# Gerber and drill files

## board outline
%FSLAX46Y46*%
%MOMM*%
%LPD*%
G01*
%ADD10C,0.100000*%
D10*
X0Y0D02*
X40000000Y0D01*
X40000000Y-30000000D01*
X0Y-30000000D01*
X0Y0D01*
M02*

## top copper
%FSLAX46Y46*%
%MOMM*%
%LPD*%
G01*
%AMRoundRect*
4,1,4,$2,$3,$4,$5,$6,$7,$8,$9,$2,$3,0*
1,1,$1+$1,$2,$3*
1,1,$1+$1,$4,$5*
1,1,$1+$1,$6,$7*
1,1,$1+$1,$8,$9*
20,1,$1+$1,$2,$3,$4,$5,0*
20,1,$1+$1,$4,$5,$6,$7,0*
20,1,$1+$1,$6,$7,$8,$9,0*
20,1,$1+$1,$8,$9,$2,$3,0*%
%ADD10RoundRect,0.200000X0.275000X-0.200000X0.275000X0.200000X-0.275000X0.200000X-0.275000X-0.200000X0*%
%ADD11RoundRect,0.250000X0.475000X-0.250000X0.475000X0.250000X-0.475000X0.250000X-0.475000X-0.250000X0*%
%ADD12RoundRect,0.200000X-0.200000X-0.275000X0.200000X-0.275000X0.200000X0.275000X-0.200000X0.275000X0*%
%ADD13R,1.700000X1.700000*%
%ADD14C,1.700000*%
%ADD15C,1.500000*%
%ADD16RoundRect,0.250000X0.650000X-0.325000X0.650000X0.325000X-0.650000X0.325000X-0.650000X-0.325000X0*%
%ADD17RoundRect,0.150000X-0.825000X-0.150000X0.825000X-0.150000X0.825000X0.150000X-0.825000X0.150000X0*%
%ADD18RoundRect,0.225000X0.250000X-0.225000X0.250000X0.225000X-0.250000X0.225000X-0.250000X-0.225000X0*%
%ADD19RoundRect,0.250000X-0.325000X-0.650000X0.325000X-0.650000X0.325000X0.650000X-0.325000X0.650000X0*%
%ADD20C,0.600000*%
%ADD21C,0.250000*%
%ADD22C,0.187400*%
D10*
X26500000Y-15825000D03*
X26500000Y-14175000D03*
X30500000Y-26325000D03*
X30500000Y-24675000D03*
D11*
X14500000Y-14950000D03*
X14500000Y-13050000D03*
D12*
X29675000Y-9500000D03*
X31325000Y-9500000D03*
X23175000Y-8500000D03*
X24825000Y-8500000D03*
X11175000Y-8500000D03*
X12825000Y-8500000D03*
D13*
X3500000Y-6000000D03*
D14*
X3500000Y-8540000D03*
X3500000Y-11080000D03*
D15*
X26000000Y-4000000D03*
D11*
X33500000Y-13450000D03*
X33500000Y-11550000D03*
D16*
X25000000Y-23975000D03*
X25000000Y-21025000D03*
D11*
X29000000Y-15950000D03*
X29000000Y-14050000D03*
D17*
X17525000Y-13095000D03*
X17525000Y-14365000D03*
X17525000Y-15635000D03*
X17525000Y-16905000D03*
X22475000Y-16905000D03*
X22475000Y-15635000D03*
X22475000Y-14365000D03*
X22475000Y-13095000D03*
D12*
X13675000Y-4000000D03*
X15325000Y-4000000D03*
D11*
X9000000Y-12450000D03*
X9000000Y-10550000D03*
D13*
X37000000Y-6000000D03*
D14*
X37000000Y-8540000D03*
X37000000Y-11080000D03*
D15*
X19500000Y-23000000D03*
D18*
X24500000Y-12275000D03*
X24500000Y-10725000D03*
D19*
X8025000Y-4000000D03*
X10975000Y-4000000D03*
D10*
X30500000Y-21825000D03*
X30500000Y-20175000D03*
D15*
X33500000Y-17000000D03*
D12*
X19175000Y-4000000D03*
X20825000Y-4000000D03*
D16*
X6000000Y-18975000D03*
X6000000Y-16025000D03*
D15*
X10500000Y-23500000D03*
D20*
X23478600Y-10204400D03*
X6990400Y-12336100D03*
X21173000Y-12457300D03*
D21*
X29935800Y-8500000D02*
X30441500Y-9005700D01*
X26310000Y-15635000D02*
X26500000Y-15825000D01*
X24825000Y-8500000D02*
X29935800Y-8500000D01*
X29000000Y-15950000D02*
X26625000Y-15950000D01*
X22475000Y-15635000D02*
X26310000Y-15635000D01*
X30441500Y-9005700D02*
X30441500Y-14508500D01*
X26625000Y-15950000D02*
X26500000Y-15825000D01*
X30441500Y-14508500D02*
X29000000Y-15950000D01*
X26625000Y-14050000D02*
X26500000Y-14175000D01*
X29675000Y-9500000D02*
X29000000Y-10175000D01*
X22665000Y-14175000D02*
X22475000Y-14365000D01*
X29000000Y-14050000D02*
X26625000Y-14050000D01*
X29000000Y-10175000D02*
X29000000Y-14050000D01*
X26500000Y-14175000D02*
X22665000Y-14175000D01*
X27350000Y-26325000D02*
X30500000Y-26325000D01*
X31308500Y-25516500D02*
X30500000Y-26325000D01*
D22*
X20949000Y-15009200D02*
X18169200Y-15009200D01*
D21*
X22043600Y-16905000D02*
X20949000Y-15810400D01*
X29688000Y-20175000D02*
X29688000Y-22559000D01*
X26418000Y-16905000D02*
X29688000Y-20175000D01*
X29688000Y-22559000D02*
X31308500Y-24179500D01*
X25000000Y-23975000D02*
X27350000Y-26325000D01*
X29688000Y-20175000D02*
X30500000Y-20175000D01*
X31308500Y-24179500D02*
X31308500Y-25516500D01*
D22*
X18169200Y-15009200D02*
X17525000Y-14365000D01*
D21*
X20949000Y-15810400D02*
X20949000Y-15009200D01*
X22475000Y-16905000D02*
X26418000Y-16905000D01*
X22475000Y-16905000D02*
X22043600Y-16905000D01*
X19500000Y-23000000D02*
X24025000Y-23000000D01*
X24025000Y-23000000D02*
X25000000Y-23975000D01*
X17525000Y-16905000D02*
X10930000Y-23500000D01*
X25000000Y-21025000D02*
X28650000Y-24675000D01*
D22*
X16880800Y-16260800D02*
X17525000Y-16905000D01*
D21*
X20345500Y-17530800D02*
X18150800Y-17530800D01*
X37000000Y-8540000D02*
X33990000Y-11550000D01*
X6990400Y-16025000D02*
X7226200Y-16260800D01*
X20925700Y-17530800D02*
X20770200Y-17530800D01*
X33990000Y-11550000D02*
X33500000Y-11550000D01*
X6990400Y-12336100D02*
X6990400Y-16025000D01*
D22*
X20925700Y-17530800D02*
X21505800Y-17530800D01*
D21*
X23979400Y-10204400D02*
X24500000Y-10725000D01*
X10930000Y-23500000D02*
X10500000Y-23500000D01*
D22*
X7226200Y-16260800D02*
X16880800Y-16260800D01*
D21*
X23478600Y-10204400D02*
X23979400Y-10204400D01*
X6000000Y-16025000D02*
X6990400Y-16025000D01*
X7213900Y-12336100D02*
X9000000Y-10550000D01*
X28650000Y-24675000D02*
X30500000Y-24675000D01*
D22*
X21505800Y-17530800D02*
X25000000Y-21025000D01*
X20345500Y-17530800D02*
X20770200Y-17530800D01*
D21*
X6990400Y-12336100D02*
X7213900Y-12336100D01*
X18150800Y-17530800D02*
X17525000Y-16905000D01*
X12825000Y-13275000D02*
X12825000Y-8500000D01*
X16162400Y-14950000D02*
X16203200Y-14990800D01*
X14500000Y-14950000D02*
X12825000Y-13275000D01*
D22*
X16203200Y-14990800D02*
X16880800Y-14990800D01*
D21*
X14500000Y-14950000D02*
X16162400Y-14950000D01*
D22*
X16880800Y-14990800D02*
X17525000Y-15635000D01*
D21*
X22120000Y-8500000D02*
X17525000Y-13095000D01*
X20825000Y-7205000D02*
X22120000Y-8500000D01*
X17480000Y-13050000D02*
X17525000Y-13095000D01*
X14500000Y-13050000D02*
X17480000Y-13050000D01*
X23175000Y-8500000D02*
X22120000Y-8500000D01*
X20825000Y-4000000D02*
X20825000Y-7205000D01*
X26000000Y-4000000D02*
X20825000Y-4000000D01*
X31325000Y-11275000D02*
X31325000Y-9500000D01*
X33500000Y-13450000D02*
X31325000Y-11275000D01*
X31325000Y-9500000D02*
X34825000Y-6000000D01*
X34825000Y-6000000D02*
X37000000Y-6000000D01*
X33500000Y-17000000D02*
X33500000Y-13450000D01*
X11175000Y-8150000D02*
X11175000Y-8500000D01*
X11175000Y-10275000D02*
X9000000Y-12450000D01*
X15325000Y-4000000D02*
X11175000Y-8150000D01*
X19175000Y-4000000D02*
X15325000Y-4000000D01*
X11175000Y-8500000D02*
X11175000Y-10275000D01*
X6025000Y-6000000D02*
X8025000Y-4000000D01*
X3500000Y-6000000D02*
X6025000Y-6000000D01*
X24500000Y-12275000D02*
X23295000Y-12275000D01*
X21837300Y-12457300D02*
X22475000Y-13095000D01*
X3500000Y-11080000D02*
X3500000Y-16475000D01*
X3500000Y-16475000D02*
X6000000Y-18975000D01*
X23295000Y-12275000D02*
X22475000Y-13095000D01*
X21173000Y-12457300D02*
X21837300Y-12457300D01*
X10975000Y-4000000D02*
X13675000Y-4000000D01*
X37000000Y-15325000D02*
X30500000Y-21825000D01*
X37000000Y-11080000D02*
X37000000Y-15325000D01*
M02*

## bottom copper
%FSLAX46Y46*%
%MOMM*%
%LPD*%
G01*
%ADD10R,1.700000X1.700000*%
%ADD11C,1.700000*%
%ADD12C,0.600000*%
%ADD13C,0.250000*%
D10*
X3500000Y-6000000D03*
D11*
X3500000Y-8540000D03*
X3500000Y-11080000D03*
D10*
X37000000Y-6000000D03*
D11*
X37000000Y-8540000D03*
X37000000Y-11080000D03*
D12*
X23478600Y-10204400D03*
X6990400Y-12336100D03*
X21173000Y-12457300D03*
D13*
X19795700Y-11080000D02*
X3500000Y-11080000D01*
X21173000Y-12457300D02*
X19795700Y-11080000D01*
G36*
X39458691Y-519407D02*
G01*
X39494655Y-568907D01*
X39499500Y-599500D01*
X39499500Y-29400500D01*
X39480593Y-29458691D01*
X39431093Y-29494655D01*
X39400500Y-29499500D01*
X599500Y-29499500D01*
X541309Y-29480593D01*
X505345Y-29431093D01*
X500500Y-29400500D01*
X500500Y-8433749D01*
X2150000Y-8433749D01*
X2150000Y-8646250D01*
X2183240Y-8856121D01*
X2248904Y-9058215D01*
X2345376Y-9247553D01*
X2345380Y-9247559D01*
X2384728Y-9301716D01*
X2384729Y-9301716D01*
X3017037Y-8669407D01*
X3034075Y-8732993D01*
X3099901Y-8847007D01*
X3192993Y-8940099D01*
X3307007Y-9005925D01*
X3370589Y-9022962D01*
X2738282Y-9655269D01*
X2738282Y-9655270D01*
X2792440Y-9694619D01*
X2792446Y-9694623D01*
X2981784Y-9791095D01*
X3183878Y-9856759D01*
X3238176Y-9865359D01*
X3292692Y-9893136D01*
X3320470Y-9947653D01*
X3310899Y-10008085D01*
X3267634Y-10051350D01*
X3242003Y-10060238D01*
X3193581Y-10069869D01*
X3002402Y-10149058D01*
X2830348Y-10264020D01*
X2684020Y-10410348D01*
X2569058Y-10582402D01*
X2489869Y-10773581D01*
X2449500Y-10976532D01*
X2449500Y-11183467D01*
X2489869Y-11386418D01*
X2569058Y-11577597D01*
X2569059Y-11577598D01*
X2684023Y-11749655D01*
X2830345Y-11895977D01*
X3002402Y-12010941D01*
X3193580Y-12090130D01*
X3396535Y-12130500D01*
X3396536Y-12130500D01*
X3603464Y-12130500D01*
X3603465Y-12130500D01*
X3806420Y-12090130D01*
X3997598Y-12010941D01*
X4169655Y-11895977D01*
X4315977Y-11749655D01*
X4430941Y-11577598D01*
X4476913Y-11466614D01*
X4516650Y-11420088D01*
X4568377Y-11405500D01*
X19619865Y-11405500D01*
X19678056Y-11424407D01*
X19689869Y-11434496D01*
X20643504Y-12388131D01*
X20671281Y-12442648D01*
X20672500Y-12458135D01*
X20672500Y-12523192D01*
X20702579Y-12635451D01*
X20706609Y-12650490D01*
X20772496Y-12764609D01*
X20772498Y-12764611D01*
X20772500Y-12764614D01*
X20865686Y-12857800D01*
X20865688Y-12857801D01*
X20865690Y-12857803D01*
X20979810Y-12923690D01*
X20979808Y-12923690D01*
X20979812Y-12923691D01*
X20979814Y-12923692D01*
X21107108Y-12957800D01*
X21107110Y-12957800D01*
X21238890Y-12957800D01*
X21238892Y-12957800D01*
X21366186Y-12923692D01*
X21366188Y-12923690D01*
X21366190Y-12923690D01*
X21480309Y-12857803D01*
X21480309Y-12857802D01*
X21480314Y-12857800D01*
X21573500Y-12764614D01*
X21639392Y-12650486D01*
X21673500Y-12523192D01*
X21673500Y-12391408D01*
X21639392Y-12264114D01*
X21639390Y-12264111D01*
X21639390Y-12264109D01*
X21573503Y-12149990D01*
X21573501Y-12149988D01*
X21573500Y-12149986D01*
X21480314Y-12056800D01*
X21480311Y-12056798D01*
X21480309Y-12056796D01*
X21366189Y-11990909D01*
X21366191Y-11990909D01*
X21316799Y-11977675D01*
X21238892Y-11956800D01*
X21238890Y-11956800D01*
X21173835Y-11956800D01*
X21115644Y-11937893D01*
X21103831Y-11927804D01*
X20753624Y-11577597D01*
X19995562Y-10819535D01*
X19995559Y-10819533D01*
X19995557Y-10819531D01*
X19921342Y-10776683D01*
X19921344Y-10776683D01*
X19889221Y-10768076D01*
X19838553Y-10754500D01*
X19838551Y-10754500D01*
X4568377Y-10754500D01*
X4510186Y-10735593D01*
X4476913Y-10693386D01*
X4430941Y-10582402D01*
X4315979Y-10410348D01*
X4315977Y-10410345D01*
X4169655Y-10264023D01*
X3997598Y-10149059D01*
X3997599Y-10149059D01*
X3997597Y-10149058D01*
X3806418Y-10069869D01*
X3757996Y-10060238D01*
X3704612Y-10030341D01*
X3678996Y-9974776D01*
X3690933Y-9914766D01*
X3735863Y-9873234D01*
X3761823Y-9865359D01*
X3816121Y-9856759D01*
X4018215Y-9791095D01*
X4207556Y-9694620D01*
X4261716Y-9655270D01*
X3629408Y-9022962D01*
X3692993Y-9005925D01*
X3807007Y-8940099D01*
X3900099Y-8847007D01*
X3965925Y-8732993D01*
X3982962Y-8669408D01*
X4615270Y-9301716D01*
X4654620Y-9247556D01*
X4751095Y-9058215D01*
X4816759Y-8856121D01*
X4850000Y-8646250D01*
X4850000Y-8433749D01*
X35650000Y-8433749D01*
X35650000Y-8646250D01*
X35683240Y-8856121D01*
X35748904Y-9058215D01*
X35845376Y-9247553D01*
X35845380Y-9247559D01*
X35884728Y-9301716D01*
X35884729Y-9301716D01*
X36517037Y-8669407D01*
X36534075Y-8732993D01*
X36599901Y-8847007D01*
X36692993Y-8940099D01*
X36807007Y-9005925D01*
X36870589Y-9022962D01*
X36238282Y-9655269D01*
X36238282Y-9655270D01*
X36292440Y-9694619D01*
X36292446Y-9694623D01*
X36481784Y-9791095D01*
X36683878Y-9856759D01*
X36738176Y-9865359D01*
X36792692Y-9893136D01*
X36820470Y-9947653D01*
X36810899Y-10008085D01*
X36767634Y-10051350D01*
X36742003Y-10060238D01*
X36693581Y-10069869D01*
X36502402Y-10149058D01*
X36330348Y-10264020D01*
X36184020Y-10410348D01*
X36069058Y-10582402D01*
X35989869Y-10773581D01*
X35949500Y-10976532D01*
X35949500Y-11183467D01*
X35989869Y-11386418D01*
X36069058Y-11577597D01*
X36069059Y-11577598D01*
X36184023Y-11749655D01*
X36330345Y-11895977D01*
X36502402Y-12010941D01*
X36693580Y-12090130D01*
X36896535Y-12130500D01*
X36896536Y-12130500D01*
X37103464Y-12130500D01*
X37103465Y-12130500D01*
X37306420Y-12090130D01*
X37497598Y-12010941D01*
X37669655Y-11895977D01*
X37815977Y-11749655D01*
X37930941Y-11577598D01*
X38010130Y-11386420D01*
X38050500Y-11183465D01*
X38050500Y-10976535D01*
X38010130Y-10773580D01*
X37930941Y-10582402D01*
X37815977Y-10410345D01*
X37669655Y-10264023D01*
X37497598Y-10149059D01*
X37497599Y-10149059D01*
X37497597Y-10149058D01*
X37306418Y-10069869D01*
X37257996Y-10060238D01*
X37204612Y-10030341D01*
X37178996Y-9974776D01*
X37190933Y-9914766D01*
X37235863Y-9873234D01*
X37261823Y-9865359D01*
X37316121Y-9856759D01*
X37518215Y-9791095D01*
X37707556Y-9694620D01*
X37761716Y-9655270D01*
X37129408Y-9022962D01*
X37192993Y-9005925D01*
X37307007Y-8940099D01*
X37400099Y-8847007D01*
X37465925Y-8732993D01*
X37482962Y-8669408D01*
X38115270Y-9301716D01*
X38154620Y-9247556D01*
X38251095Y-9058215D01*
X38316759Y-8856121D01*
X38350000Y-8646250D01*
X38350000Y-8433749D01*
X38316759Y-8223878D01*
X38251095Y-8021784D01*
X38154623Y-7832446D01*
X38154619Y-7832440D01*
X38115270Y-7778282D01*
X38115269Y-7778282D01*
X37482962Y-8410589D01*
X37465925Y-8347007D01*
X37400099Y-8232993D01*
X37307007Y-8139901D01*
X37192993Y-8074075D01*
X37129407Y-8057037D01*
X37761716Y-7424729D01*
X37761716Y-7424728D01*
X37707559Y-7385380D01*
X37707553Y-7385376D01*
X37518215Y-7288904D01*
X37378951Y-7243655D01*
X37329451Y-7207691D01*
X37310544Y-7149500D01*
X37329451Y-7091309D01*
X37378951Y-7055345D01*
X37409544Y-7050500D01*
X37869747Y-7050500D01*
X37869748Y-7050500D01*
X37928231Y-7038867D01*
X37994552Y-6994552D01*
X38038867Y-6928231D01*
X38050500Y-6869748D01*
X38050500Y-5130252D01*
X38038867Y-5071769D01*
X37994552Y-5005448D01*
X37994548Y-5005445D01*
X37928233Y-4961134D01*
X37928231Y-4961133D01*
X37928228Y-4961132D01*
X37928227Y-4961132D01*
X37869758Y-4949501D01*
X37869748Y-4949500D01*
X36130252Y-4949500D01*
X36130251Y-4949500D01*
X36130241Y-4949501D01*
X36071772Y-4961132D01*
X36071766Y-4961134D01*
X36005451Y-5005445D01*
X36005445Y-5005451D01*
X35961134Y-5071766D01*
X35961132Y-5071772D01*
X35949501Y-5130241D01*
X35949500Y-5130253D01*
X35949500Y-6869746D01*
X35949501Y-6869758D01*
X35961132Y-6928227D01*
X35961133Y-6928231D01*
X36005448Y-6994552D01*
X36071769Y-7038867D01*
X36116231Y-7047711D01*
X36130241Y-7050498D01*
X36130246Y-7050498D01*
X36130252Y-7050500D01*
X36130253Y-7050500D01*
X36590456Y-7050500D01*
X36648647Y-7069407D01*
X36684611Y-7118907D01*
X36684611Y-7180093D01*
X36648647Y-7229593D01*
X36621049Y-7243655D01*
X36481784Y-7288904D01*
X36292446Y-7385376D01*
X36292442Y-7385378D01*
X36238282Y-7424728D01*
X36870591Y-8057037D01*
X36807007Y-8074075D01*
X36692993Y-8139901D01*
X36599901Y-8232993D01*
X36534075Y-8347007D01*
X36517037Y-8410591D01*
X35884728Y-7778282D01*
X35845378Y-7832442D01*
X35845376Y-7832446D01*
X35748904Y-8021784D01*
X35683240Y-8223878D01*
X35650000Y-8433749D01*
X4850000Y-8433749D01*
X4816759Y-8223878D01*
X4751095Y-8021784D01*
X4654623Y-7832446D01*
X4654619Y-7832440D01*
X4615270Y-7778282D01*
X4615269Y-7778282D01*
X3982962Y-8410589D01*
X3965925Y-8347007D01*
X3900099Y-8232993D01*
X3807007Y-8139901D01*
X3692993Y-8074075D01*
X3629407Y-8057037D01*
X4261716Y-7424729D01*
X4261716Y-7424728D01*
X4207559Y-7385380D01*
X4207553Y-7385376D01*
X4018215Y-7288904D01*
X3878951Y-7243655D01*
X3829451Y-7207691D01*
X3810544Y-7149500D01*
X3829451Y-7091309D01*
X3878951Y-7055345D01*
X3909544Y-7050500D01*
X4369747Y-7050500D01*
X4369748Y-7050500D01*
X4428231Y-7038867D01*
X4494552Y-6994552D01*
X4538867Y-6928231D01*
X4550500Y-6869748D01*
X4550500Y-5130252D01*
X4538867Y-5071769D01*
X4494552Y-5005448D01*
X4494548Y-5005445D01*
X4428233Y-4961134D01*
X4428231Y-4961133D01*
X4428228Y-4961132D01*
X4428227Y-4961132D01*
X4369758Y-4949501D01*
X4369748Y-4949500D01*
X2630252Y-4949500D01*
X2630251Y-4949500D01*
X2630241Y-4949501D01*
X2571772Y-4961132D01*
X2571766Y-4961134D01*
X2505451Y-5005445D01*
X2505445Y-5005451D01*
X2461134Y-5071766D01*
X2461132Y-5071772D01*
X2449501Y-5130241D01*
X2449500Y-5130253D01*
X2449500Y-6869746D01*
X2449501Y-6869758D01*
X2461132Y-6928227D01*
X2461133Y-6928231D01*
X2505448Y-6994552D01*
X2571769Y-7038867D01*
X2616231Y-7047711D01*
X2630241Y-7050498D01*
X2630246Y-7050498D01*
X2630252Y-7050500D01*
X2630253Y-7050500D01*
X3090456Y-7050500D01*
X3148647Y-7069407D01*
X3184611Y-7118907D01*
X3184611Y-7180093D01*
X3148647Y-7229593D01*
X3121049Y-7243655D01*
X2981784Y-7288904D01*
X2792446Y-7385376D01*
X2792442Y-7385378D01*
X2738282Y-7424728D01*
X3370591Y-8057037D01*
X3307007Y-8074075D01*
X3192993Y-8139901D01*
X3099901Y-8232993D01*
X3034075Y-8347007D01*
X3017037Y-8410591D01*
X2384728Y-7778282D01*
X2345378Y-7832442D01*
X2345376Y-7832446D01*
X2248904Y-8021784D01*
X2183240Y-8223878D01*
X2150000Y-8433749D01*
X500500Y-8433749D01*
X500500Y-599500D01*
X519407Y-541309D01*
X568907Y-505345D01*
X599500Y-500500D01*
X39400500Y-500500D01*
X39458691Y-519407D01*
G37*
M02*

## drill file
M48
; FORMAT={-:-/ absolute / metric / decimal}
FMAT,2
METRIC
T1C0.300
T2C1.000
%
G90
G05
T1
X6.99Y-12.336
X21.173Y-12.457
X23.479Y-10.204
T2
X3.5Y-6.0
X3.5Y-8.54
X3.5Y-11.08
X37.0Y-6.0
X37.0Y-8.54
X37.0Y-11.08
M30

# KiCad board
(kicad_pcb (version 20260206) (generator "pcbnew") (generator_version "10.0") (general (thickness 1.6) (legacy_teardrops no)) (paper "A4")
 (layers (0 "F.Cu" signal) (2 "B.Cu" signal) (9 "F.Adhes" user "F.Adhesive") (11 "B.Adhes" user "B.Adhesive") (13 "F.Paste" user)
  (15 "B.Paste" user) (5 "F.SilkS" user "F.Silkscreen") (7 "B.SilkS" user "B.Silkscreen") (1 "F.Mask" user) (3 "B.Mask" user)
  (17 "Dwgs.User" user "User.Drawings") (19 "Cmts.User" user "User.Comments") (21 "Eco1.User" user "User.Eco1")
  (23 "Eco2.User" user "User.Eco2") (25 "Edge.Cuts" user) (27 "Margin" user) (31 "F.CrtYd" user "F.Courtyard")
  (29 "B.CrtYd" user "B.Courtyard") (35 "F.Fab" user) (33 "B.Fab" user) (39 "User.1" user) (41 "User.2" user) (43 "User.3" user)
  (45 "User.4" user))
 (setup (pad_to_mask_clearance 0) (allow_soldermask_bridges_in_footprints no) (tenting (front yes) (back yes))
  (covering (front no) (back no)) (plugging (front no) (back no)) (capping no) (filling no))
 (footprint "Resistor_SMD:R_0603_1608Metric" (layer "F.Cu") (at 26.5 15 90)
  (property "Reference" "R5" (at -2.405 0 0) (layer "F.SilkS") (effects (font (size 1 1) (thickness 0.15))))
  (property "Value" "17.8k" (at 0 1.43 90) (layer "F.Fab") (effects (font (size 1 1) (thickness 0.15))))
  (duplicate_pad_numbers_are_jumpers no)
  (pad "1" smd roundrect (at -0.825 0 90) (size 0.8 0.95) (layers "F.Cu" "F.Mask" "F.Paste") (roundrect_rratio 0.25) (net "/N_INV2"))
  (pad "2" smd roundrect (at 0.825 0 90) (size 0.8 0.95) (layers "F.Cu" "F.Mask" "F.Paste") (roundrect_rratio 0.25) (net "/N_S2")))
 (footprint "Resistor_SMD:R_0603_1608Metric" (layer "F.Cu") (at 30.5 25.5 90)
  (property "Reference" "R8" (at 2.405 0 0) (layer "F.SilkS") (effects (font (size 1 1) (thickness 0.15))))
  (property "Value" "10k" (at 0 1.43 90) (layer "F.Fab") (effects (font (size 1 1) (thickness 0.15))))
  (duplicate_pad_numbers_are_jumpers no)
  (pad "1" smd roundrect (at -0.825 0 90) (size 0.8 0.95) (layers "F.Cu" "F.Mask" "F.Paste") (roundrect_rratio 0.25) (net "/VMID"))
  (pad "2" smd roundrect (at 0.825 0 90) (size 0.8 0.95) (layers "F.Cu" "F.Mask" "F.Paste") (roundrect_rratio 0.25) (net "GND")))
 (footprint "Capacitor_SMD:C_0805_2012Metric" (layer "F.Cu") (at 14.5 14 90)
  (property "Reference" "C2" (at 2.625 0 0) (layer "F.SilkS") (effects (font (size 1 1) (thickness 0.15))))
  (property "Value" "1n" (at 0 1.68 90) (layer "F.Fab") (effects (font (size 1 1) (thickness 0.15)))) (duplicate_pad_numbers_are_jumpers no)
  (pad "1" smd roundrect (at -0.95 0 90) (size 1 1.45) (layers "F.Cu" "F.Mask" "F.Paste") (roundrect_rratio 0.25) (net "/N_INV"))
  (pad "2" smd roundrect (at 0.95 0 90) (size 1 1.45) (layers "F.Cu" "F.Mask" "F.Paste") (roundrect_rratio 0.25) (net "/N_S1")))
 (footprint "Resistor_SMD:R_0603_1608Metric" (layer "F.Cu") (at 30.5 9.5)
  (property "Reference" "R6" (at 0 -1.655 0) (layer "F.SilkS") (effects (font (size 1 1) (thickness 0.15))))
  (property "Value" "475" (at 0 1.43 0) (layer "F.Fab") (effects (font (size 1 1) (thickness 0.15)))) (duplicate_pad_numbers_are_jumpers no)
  (pad "1" smd roundrect (at -0.825 0) (size 0.8 0.95) (layers "F.Cu" "F.Mask" "F.Paste") (roundrect_rratio 0.25) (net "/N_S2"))
  (pad "2" smd roundrect (at 0.825 0) (size 0.8 0.95) (layers "F.Cu" "F.Mask" "F.Paste") (roundrect_rratio 0.25) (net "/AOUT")))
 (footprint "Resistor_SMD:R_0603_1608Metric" (layer "F.Cu") (at 24 8.5)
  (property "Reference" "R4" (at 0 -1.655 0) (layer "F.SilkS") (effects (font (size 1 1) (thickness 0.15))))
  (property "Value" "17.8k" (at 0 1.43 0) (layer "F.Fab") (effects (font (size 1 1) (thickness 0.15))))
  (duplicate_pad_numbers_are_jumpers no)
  (pad "1" smd roundrect (at -0.825 0) (size 0.8 0.95) (layers "F.Cu" "F.Mask" "F.Paste") (roundrect_rratio 0.25) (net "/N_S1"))
  (pad "2" smd roundrect (at 0.825 0) (size 0.8 0.95) (layers "F.Cu" "F.Mask" "F.Paste") (roundrect_rratio 0.25) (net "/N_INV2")))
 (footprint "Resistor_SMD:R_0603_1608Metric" (layer "F.Cu") (at 12 8.5)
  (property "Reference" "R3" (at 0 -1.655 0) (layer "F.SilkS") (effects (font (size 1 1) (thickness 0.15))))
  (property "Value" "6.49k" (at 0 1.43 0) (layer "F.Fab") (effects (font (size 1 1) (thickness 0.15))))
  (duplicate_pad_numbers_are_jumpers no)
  (pad "1" smd roundrect (at -0.825 0) (size 0.8 0.95) (layers "F.Cu" "F.Mask" "F.Paste") (roundrect_rratio 0.25) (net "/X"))
  (pad "2" smd roundrect (at 0.825 0) (size 0.8 0.95) (layers "F.Cu" "F.Mask" "F.Paste") (roundrect_rratio 0.25) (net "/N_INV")))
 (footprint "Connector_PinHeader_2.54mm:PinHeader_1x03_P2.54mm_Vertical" (layer "F.Cu") (at 3.5 6)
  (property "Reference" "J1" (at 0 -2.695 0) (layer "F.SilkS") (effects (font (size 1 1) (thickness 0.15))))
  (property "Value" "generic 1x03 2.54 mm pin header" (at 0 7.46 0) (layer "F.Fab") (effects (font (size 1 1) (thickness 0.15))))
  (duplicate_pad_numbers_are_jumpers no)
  (pad "1" thru_hole rect (at 0 0) (size 1.7 1.7) (drill 1) (layers "*.Cu" "*.Mask") (remove_unused_layers no) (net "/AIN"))
  (pad "2" thru_hole circle (at 0 2.54) (size 1.7 1.7) (drill 1) (layers "*.Cu" "*.Mask") (remove_unused_layers no) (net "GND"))
  (pad "3" thru_hole circle (at 0 5.08) (size 1.7 1.7) (drill 1) (layers "*.Cu" "*.Mask") (remove_unused_layers no) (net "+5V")))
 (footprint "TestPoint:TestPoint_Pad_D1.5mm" (layer "F.Cu") (at 26 4)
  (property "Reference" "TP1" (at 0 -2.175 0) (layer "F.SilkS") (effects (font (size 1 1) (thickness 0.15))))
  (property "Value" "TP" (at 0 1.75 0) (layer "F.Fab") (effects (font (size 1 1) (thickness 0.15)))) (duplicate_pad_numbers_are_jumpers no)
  (pad "1" smd circle (at 0 0) (size 1.5 1.5) (layers "F.Cu" "F.Mask") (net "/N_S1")))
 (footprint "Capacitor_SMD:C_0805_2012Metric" (layer "F.Cu") (at 33.5 12.5 90)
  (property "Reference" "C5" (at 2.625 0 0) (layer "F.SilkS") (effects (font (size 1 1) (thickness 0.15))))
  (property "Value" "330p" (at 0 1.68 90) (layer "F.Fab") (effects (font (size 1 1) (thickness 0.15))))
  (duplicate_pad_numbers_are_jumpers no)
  (pad "1" smd roundrect (at -0.95 0 90) (size 1 1.45) (layers "F.Cu" "F.Mask" "F.Paste") (roundrect_rratio 0.25) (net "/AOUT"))
  (pad "2" smd roundrect (at 0.95 0 90) (size 1 1.45) (layers "F.Cu" "F.Mask" "F.Paste") (roundrect_rratio 0.25) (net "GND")))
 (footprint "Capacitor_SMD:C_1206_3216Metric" (layer "F.Cu") (at 25 22.5 90)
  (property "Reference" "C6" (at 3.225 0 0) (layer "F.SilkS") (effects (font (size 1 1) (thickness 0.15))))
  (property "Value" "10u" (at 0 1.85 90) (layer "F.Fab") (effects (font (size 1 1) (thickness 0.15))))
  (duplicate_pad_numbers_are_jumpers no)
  (pad "1" smd roundrect (at -1.475 0 90) (size 1.15 1.8) (layers "F.Cu" "F.Mask" "F.Paste") (roundrect_rratio 0.217391) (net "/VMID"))
  (pad "2" smd roundrect (at 1.475 0 90) (size 1.15 1.8) (layers "F.Cu" "F.Mask" "F.Paste") (roundrect_rratio 0.217391) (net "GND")))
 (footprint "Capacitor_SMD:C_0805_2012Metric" (layer "F.Cu") (at 29 15 90)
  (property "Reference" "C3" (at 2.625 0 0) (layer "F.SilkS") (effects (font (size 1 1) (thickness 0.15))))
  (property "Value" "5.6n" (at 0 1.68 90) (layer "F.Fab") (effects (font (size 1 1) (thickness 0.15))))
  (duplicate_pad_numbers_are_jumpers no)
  (pad "1" smd roundrect (at -0.95 0 90) (size 1 1.45) (layers "F.Cu" "F.Mask" "F.Paste") (roundrect_rratio 0.25) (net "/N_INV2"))
  (pad "2" smd roundrect (at 0.95 0 90) (size 1 1.45) (layers "F.Cu" "F.Mask" "F.Paste") (roundrect_rratio 0.25) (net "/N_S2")))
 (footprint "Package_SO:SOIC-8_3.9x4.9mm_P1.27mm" (layer "F.Cu") (at 20 15)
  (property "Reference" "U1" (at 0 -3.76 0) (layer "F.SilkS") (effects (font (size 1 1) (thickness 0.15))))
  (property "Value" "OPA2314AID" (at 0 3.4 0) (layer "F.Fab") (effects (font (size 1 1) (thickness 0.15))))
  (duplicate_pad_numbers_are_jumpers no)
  (pad "1" smd roundrect (at -2.475 -1.905) (size 1.95 0.6) (layers "F.Cu" "F.Mask" "F.Paste") (roundrect_rratio 0.25) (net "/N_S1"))
  (pad "2" smd roundrect (at -2.475 -0.635) (size 1.95 0.6) (layers "F.Cu" "F.Mask" "F.Paste") (roundrect_rratio 0.25) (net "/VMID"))
  (pad "3" smd roundrect (at -2.475 0.635) (size 1.95 0.6) (layers "F.Cu" "F.Mask" "F.Paste") (roundrect_rratio 0.25) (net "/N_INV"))
  (pad "4" smd roundrect (at -2.475 1.905) (size 1.95 0.6) (layers "F.Cu" "F.Mask" "F.Paste") (roundrect_rratio 0.25) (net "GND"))
  (pad "5" smd roundrect (at 2.475 1.905) (size 1.95 0.6) (layers "F.Cu" "F.Mask" "F.Paste") (roundrect_rratio 0.25) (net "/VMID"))
  (pad "6" smd roundrect (at 2.475 0.635) (size 1.95 0.6) (layers "F.Cu" "F.Mask" "F.Paste") (roundrect_rratio 0.25) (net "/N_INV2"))
  (pad "7" smd roundrect (at 2.475 -0.635) (size 1.95 0.6) (layers "F.Cu" "F.Mask" "F.Paste") (roundrect_rratio 0.25) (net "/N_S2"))
  (pad "8" smd roundrect (at 2.475 -1.905) (size 1.95 0.6) (layers "F.Cu" "F.Mask" "F.Paste") (roundrect_rratio 0.25) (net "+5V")))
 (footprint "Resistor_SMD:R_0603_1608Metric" (layer "F.Cu") (at 14.5 4)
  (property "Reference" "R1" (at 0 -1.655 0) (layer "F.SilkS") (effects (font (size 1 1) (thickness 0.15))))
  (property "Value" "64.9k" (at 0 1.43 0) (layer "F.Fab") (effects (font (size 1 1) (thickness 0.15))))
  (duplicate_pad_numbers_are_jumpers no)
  (pad "1" smd roundrect (at -0.825 0) (size 0.8 0.95) (layers "F.Cu" "F.Mask" "F.Paste") (roundrect_rratio 0.25) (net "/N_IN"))
  (pad "2" smd roundrect (at 0.825 0) (size 0.8 0.95) (layers "F.Cu" "F.Mask" "F.Paste") (roundrect_rratio 0.25) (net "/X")))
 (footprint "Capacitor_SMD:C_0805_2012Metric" (layer "F.Cu") (at 9 11.5 90)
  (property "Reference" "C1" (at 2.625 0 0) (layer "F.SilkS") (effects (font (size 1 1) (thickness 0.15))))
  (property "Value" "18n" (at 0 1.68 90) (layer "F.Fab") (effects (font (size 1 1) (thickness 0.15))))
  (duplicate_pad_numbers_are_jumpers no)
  (pad "1" smd roundrect (at -0.95 0 90) (size 1 1.45) (layers "F.Cu" "F.Mask" "F.Paste") (roundrect_rratio 0.25) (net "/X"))
  (pad "2" smd roundrect (at 0.95 0 90) (size 1 1.45) (layers "F.Cu" "F.Mask" "F.Paste") (roundrect_rratio 0.25) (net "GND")))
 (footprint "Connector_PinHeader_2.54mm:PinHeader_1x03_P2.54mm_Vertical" (layer "F.Cu") (at 37 6)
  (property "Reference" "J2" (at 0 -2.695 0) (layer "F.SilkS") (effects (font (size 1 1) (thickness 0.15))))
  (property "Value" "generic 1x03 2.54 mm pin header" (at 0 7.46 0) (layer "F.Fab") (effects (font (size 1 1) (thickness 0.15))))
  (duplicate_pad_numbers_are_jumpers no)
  (pad "1" thru_hole rect (at 0 0) (size 1.7 1.7) (drill 1) (layers "*.Cu" "*.Mask") (remove_unused_layers no) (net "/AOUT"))
  (pad "2" thru_hole circle (at 0 2.54) (size 1.7 1.7) (drill 1) (layers "*.Cu" "*.Mask") (remove_unused_layers no) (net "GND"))
  (pad "3" thru_hole circle (at 0 5.08) (size 1.7 1.7) (drill 1) (layers "*.Cu" "*.Mask") (remove_unused_layers no) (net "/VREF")))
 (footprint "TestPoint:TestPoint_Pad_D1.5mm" (layer "F.Cu") (at 19.5 23)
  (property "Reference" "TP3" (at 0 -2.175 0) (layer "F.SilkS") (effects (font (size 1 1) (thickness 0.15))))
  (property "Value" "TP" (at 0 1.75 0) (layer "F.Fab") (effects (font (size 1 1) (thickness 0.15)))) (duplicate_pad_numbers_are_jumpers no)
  (pad "1" smd circle (at 0 0) (size 1.5 1.5) (layers "F.Cu" "F.Mask") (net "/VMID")))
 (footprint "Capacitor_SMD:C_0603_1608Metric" (layer "F.Cu") (at 24.5 11.5 90)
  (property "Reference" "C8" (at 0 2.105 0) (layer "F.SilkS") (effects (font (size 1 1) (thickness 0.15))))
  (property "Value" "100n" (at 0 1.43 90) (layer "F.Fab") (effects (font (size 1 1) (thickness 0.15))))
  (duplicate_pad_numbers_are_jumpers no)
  (pad "1" smd roundrect (at -0.775 0 90) (size 0.9 0.95) (layers "F.Cu" "F.Mask" "F.Paste") (roundrect_rratio 0.25) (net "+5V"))
  (pad "2" smd roundrect (at 0.775 0 90) (size 0.9 0.95) (layers "F.Cu" "F.Mask" "F.Paste") (roundrect_rratio 0.25) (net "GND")))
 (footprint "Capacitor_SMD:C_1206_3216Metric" (layer "F.Cu") (at 9.5 4)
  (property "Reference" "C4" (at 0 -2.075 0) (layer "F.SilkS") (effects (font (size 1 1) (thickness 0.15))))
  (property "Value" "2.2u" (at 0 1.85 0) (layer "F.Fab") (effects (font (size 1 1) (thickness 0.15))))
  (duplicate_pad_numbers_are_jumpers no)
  (pad "1" smd roundrect (at -1.475 0) (size 1.15 1.8) (layers "F.Cu" "F.Mask" "F.Paste") (roundrect_rratio 0.217391) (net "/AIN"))
  (pad "2" smd roundrect (at 1.475 0) (size 1.15 1.8) (layers "F.Cu" "F.Mask" "F.Paste") (roundrect_rratio 0.217391) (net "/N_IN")))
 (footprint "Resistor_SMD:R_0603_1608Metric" (layer "F.Cu") (at 30.5 21 90)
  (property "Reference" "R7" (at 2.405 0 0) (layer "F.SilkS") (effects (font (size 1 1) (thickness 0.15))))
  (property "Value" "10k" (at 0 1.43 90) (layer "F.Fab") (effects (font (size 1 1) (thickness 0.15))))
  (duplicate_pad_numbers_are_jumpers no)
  (pad "1" smd roundrect (at -0.825 0 90) (size 0.8 0.95) (layers "F.Cu" "F.Mask" "F.Paste") (roundrect_rratio 0.25) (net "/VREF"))
  (pad "2" smd roundrect (at 0.825 0 90) (size 0.8 0.95) (layers "F.Cu" "F.Mask" "F.Paste") (roundrect_rratio 0.25) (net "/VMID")))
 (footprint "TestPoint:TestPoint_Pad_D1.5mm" (layer "F.Cu") (at 33.5 17)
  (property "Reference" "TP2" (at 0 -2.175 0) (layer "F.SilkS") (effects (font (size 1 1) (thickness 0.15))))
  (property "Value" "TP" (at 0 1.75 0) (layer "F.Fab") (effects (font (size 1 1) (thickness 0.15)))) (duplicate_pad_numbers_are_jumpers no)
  (pad "1" smd circle (at 0 0) (size 1.5 1.5) (layers "F.Cu" "F.Mask") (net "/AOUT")))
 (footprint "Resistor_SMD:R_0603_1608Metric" (layer "F.Cu") (at 20 4)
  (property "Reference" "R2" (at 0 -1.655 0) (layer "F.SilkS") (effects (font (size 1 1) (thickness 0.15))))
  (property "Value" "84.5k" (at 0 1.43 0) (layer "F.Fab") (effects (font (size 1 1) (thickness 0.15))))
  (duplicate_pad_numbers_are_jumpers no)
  (pad "1" smd roundrect (at -0.825 0) (size 0.8 0.95) (layers "F.Cu" "F.Mask" "F.Paste") (roundrect_rratio 0.25) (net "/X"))
  (pad "2" smd roundrect (at 0.825 0) (size 0.8 0.95) (layers "F.Cu" "F.Mask" "F.Paste") (roundrect_rratio 0.25) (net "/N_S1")))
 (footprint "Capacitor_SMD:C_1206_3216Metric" (layer "F.Cu") (at 6 17.5 90)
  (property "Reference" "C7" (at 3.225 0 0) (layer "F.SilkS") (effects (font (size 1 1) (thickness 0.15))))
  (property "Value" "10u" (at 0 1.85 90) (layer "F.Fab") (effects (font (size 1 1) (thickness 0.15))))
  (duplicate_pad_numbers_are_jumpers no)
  (pad "1" smd roundrect (at -1.475 0 90) (size 1.15 1.8) (layers "F.Cu" "F.Mask" "F.Paste") (roundrect_rratio 0.217391) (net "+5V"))
  (pad "2" smd roundrect (at 1.475 0 90) (size 1.15 1.8) (layers "F.Cu" "F.Mask" "F.Paste") (roundrect_rratio 0.217391) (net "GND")))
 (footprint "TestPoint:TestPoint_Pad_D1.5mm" (layer "F.Cu") (at 10.5 23.5)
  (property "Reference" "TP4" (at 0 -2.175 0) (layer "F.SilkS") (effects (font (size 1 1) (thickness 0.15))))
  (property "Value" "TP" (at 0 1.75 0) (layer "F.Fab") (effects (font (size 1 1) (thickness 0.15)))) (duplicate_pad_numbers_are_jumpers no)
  (pad "1" smd circle (at 0 0) (size 1.5 1.5) (layers "F.Cu" "F.Mask") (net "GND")))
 (gr_rect (start 0 0) (end 40 30) (stroke (width 0.1) (type default)) (fill no) (layer "Edge.Cuts"))
 (segment (start 29.9358 8.5) (end 30.4415 9.0057) (width 0.25) (layer "F.Cu") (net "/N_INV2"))
 (segment (start 26.31 15.635) (end 26.5 15.825) (width 0.25) (layer "F.Cu") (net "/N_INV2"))
 (segment (start 24.825 8.5) (end 29.9358 8.5) (width 0.25) (layer "F.Cu") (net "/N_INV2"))
 (segment (start 29 15.95) (end 26.625 15.95) (width 0.25) (layer "F.Cu") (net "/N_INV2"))
 (segment (start 22.475 15.635) (end 26.31 15.635) (width 0.25) (layer "F.Cu") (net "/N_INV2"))
 (segment (start 30.4415 9.0057) (end 30.4415 14.5085) (width 0.25) (layer "F.Cu") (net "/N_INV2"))
 (segment (start 26.625 15.95) (end 26.5 15.825) (width 0.25) (layer "F.Cu") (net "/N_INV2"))
 (segment (start 30.4415 14.5085) (end 29 15.95) (width 0.25) (layer "F.Cu") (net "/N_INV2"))
 (segment (start 26.625 14.05) (end 26.5 14.175) (width 0.25) (layer "F.Cu") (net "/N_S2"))
 (segment (start 29.675 9.5) (end 29 10.175) (width 0.25) (layer "F.Cu") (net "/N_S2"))
 (segment (start 22.665 14.175) (end 22.475 14.365) (width 0.25) (layer "F.Cu") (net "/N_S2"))
 (segment (start 29 14.05) (end 26.625 14.05) (width 0.25) (layer "F.Cu") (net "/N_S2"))
 (segment (start 29 10.175) (end 29 14.05) (width 0.25) (layer "F.Cu") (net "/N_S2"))
 (segment (start 26.5 14.175) (end 22.665 14.175) (width 0.25) (layer "F.Cu") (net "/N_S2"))
 (segment (start 27.35 26.325) (end 30.5 26.325) (width 0.25) (layer "F.Cu") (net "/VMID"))
 (segment (start 31.3085 25.5165) (end 30.5 26.325) (width 0.25) (layer "F.Cu") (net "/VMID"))
 (segment (start 20.949 15.0092) (end 18.1692 15.0092) (width 0.1874) (layer "F.Cu") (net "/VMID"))
 (segment (start 22.0436 16.905) (end 20.949 15.8104) (width 0.25) (layer "F.Cu") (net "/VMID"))
 (segment (start 29.688 20.175) (end 29.688 22.559) (width 0.25) (layer "F.Cu") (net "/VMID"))
 (segment (start 26.418 16.905) (end 29.688 20.175) (width 0.25) (layer "F.Cu") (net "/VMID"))
 (segment (start 29.688 22.559) (end 31.3085 24.1795) (width 0.25) (layer "F.Cu") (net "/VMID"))
 (segment (start 25 23.975) (end 27.35 26.325) (width 0.25) (layer "F.Cu") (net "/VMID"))
 (segment (start 29.688 20.175) (end 30.5 20.175) (width 0.25) (layer "F.Cu") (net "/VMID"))
 (segment (start 31.3085 24.1795) (end 31.3085 25.5165) (width 0.25) (layer "F.Cu") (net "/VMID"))
 (segment (start 18.1692 15.0092) (end 17.525 14.365) (width 0.1874) (layer "F.Cu") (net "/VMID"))
 (segment (start 20.949 15.8104) (end 20.949 15.0092) (width 0.25) (layer "F.Cu") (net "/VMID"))
 (segment (start 22.475 16.905) (end 26.418 16.905) (width 0.25) (layer "F.Cu") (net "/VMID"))
 (segment (start 22.475 16.905) (end 22.0436 16.905) (width 0.25) (layer "F.Cu") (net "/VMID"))
 (segment (start 19.5 23) (end 24.025 23) (width 0.25) (layer "F.Cu") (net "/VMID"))
 (segment (start 24.025 23) (end 25 23.975) (width 0.25) (layer "F.Cu") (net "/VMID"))
 (segment (start 17.525 16.905) (end 10.93 23.5) (width 0.25) (layer "F.Cu") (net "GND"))
 (segment (start 25 21.025) (end 28.65 24.675) (width 0.25) (layer "F.Cu") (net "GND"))
 (segment (start 16.8808 16.2608) (end 17.525 16.905) (width 0.1874) (layer "F.Cu") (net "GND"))
 (segment (start 20.3455 17.5308) (end 18.1508 17.5308) (width 0.25) (layer "F.Cu") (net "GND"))
 (segment (start 37 8.54) (end 33.99 11.55) (width 0.25) (layer "F.Cu") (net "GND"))
 (segment (start 6.9904 16.025) (end 7.2262 16.2608) (width 0.25) (layer "F.Cu") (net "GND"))
 (segment (start 20.9257 17.5308) (end 20.7702 17.5308) (width 0.25) (layer "F.Cu") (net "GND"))
 (segment (start 33.99 11.55) (end 33.5 11.55) (width 0.25) (layer "F.Cu") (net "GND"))
 (segment (start 6.9904 12.3361) (end 6.9904 16.025) (width 0.25) (layer "F.Cu") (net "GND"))
 (segment (start 20.9257 17.5308) (end 21.5058 17.5308) (width 0.1874) (layer "F.Cu") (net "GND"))
 (segment (start 23.9794 10.2044) (end 24.5 10.725) (width 0.25) (layer "F.Cu") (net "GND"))
 (segment (start 10.93 23.5) (end 10.5 23.5) (width 0.25) (layer "F.Cu") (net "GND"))
 (segment (start 7.2262 16.2608) (end 16.8808 16.2608) (width 0.1874) (layer "F.Cu") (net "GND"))
 (segment (start 23.4786 10.2044) (end 23.9794 10.2044) (width 0.25) (layer "F.Cu") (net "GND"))
 (segment (start 6 16.025) (end 6.9904 16.025) (width 0.25) (layer "F.Cu") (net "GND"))
 (segment (start 7.2139 12.3361) (end 9 10.55) (width 0.25) (layer "F.Cu") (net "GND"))
 (segment (start 28.65 24.675) (end 30.5 24.675) (width 0.25) (layer "F.Cu") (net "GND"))
 (segment (start 21.5058 17.5308) (end 25 21.025) (width 0.1874) (layer "F.Cu") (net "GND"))
 (segment (start 20.3455 17.5308) (end 20.7702 17.5308) (width 0.1874) (layer "F.Cu") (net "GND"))
 (segment (start 6.9904 12.3361) (end 7.2139 12.3361) (width 0.25) (layer "F.Cu") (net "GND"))
 (segment (start 18.1508 17.5308) (end 17.525 16.905) (width 0.25) (layer "F.Cu") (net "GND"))
 (via (at 23.4786 10.2044) (size 0.6) (drill 0.3) (layers "F.Cu" "B.Cu") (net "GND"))
 (via (at 6.9904 12.3361) (size 0.6) (drill 0.3) (layers "F.Cu" "B.Cu") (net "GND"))
 (segment (start 12.825 13.275) (end 12.825 8.5) (width 0.25) (layer "F.Cu") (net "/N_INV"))
 (segment (start 16.1624 14.95) (end 16.2032 14.9908) (width 0.25) (layer "F.Cu") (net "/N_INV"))
 (segment (start 14.5 14.95) (end 12.825 13.275) (width 0.25) (layer "F.Cu") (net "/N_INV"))
 (segment (start 16.2032 14.9908) (end 16.8808 14.9908) (width 0.1874) (layer "F.Cu") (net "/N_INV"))
 (segment (start 14.5 14.95) (end 16.1624 14.95) (width 0.25) (layer "F.Cu") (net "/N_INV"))
 (segment (start 16.8808 14.9908) (end 17.525 15.635) (width 0.1874) (layer "F.Cu") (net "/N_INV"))
 (segment (start 22.12 8.5) (end 17.525 13.095) (width 0.25) (layer "F.Cu") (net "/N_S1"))
 (segment (start 20.825 7.205) (end 22.12 8.5) (width 0.25) (layer "F.Cu") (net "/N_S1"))
 (segment (start 17.48 13.05) (end 17.525 13.095) (width 0.25) (layer "F.Cu") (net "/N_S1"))
 (segment (start 14.5 13.05) (end 17.48 13.05) (width 0.25) (layer "F.Cu") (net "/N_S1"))
 (segment (start 23.175 8.5) (end 22.12 8.5) (width 0.25) (layer "F.Cu") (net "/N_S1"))
 (segment (start 20.825 4) (end 20.825 7.205) (width 0.25) (layer "F.Cu") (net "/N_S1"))
 (segment (start 26 4) (end 20.825 4) (width 0.25) (layer "F.Cu") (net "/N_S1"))
 (segment (start 31.325 11.275) (end 31.325 9.5) (width 0.25) (layer "F.Cu") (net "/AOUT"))
 (segment (start 33.5 13.45) (end 31.325 11.275) (width 0.25) (layer "F.Cu") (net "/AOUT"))
 (segment (start 31.325 9.5) (end 34.825 6) (width 0.25) (layer "F.Cu") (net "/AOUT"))
 (segment (start 34.825 6) (end 37 6) (width 0.25) (layer "F.Cu") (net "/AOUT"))
 (segment (start 33.5 17) (end 33.5 13.45) (width 0.25) (layer "F.Cu") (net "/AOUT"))
 (segment (start 11.175 8.15) (end 11.175 8.5) (width 0.25) (layer "F.Cu") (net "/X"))
 (segment (start 11.175 10.275) (end 9 12.45) (width 0.25) (layer "F.Cu") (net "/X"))
 (segment (start 15.325 4) (end 11.175 8.15) (width 0.25) (layer "F.Cu") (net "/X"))
 (segment (start 19.175 4) (end 15.325 4) (width 0.25) (layer "F.Cu") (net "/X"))
 (segment (start 11.175 8.5) (end 11.175 10.275) (width 0.25) (layer "F.Cu") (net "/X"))
 (segment (start 6.025 6) (end 8.025 4) (width 0.25) (layer "F.Cu") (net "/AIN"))
 (segment (start 3.5 6) (end 6.025 6) (width 0.25) (layer "F.Cu") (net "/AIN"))
 (segment (start 24.5 12.275) (end 23.295 12.275) (width 0.25) (layer "F.Cu") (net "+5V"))
 (segment (start 21.8373 12.4573) (end 22.475 13.095) (width 0.25) (layer "F.Cu") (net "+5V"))
 (segment (start 3.5 11.08) (end 3.5 16.475) (width 0.25) (layer "F.Cu") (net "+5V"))
 (segment (start 3.5 16.475) (end 6 18.975) (width 0.25) (layer "F.Cu") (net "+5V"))
 (segment (start 23.295 12.275) (end 22.475 13.095) (width 0.25) (layer "F.Cu") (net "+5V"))
 (segment (start 21.173 12.4573) (end 21.8373 12.4573) (width 0.25) (layer "F.Cu") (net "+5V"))
 (via (at 21.173 12.4573) (size 0.6) (drill 0.3) (layers "F.Cu" "B.Cu") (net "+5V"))
 (segment (start 19.7957 11.08) (end 3.5 11.08) (width 0.25) (layer "B.Cu") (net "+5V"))
 (segment (start 21.173 12.4573) (end 19.7957 11.08) (width 0.25) (layer "B.Cu") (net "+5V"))
 (segment (start 10.975 4) (end 13.675 4) (width 0.25) (layer "F.Cu") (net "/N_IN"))
 (segment (start 37 15.325) (end 30.5 21.825) (width 0.25) (layer "F.Cu") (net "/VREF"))
 (segment (start 37 11.08) (end 37 15.325) (width 0.25) (layer "F.Cu") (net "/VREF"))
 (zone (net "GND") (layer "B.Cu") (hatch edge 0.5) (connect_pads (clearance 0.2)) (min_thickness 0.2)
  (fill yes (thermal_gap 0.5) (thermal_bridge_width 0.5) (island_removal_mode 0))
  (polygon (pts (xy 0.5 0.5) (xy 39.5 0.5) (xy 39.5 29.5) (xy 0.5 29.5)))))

